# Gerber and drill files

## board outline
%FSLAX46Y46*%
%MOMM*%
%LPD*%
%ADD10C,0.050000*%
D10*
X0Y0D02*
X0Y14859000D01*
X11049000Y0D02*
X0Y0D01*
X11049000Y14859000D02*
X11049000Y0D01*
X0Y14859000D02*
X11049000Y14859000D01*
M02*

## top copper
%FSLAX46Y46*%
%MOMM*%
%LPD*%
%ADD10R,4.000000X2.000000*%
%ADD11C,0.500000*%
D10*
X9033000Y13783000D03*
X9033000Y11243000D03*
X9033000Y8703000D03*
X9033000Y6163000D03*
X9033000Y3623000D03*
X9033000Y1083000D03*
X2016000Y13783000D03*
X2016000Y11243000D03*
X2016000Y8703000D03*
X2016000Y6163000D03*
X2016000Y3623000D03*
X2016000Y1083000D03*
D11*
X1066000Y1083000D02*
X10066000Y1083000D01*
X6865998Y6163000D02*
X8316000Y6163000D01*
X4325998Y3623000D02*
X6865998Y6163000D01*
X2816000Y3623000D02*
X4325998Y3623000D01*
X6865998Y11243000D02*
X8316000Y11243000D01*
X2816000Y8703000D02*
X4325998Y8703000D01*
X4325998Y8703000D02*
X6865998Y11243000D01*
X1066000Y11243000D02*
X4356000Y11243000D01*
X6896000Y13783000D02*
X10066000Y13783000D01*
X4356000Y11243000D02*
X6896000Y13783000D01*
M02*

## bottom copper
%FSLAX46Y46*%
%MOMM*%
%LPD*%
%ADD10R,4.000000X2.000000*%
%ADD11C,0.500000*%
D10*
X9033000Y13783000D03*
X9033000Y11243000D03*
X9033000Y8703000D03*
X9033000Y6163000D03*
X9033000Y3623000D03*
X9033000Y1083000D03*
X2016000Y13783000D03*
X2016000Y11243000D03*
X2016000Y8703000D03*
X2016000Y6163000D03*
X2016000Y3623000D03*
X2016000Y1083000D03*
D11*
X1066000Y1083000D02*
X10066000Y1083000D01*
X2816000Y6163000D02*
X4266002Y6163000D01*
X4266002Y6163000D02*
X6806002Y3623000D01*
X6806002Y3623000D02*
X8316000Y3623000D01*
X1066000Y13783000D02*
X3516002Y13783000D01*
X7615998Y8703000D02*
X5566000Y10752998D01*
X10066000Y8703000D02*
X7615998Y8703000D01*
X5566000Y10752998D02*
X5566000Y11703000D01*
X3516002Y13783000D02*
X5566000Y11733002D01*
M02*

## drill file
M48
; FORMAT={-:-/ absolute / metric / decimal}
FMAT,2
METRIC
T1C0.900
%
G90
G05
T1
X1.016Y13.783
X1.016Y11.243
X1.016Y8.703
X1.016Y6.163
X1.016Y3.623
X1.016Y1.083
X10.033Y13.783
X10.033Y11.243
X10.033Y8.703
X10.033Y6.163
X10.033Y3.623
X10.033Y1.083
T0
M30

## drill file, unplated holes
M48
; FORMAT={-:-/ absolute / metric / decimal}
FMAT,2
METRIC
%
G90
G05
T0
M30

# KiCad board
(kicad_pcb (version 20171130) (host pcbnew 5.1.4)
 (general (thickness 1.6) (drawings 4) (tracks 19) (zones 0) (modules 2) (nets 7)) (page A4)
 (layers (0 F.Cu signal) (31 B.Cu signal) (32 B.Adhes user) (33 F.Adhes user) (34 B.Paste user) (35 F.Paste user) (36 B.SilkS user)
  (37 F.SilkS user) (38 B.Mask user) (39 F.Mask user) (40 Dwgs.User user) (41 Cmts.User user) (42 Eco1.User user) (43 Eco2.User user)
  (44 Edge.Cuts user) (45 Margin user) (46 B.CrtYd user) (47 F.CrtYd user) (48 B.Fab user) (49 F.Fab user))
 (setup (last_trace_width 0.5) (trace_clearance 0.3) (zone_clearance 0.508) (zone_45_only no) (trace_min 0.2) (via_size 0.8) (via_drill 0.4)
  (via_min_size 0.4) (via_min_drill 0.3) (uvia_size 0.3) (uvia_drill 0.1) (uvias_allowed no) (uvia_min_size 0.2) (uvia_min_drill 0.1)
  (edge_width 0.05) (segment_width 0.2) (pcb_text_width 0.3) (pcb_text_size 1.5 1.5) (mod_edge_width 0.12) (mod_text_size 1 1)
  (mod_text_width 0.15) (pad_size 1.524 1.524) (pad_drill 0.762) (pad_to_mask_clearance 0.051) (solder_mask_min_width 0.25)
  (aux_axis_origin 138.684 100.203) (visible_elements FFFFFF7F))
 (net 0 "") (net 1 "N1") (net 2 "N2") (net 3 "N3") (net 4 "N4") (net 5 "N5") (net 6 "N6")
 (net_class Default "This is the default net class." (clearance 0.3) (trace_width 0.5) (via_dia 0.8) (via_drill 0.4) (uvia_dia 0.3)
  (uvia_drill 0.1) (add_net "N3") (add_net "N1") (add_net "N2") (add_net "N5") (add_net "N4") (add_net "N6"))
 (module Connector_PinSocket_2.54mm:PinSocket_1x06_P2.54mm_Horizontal (layer F.Cu) (at 148.717 99.12 180)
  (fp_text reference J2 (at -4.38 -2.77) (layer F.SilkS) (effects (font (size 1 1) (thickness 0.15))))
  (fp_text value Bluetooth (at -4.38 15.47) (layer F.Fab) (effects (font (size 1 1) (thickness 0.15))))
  (pad 6 thru_hole rect (at 0 12.7 180) (size 4 2) (drill 0.9 (offset 1 0)) (layers *.Cu *.Mask) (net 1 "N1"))
  (pad 5 thru_hole rect (at 0 10.16 180) (size 4 2) (drill 0.9 (offset 1 0)) (layers *.Cu *.Mask) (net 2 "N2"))
  (pad 4 thru_hole rect (at 0 7.62 180) (size 4 2) (drill 0.9 (offset 1 0)) (layers *.Cu *.Mask) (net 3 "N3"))
  (pad 3 thru_hole rect (at 0 5.08 180) (size 4 2) (drill 0.9 (offset 1 0)) (layers *.Cu *.Mask) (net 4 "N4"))
  (pad 2 thru_hole rect (at 0 2.54 180) (size 4 2) (drill 0.9 (offset 1 0)) (layers *.Cu *.Mask) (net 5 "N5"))
  (pad 1 thru_hole rect (at 0 0 180) (size 4 2) (drill 0.9 (offset 1 0)) (layers *.Cu *.Mask) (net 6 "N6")))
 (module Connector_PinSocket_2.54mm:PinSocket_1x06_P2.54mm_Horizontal (layer F.Cu) (at 139.7 86.42)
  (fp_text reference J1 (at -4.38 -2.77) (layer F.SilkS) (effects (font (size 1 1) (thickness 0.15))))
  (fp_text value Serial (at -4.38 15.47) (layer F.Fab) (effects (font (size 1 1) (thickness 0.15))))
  (pad 1 thru_hole rect (at 0 0) (size 4 2) (drill 0.9 (offset 1 0)) (layers *.Cu *.Mask) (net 3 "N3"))
  (pad 2 thru_hole rect (at 0 2.54) (size 4 2) (drill 0.9 (offset 1 0)) (layers *.Cu *.Mask) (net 1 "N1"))
  (pad 3 thru_hole rect (at 0 5.08) (size 4 2) (drill 0.9 (offset 1 0)) (layers *.Cu *.Mask) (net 2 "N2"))
  (pad 4 thru_hole rect (at 0 7.62) (size 4 2) (drill 0.9 (offset 1 0)) (layers *.Cu *.Mask) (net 5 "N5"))
  (pad 5 thru_hole rect (at 0 10.16) (size 4 2) (drill 0.9 (offset 1 0)) (layers *.Cu *.Mask) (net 4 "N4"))
  (pad 6 thru_hole rect (at 0 12.7) (size 4 2) (drill 0.9 (offset 1 0)) (layers *.Cu *.Mask) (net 6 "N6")))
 (gr_line (start 138.684 100.203) (end 138.684 85.344) (layer Edge.Cuts) (width 0.05))
 (gr_line (start 149.733 100.203) (end 138.684 100.203) (layer Edge.Cuts) (width 0.05))
 (gr_line (start 149.733 85.344) (end 149.733 100.203) (layer Edge.Cuts) (width 0.05))
 (gr_line (start 138.684 85.344) (end 149.733 85.344) (layer Edge.Cuts) (width 0.05))
 (segment (start 139.75 99.12) (end 148.75 99.12) (width 0.5) (layer F.Cu) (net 6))
 (segment (start 139.75 99.12) (end 148.75 99.12) (width 0.5) (layer B.Cu) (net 6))
 (segment (start 145.549998 94.04) (end 147 94.04) (width 0.5) (layer F.Cu) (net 4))
 (segment (start 143.009998 96.58) (end 145.549998 94.04) (width 0.5) (layer F.Cu) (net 4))
 (segment (start 141.5 96.58) (end 143.009998 96.58) (width 0.5) (layer F.Cu) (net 4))
 (segment (start 141.5 94.04) (end 142.950002 94.04) (width 0.5) (layer B.Cu) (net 5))
 (segment (start 142.950002 94.04) (end 145.490002 96.58) (width 0.5) (layer B.Cu) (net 5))
 (segment (start 145.490002 96.58) (end 147 96.58) (width 0.5) (layer B.Cu) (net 5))
 (segment (start 145.549998 88.96) (end 147 88.96) (width 0.5) (layer F.Cu) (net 2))
 (segment (start 141.5 91.5) (end 143.009998 91.5) (width 0.5) (layer F.Cu) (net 2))
 (segment (start 143.009998 91.5) (end 145.549998 88.96) (width 0.5) (layer F.Cu) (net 2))
 (segment (start 139.75 88.96) (end 143.04 88.96) (width 0.5) (layer F.Cu) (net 1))
 (segment (start 145.58 86.42) (end 148.75 86.42) (width 0.5) (layer F.Cu) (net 1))
 (segment (start 143.04 88.96) (end 145.58 86.42) (width 0.5) (layer F.Cu) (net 1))
 (segment (start 139.75 86.42) (end 142.200002 86.42) (width 0.5) (layer B.Cu) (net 3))
 (segment (start 146.299998 91.5) (end 144.25 89.450002) (width 0.5) (layer B.Cu) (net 3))
 (segment (start 148.75 91.5) (end 146.299998 91.5) (width 0.5) (layer B.Cu) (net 3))
 (segment (start 144.25 89.450002) (end 144.25 88.5) (width 0.5) (layer B.Cu) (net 3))
 (segment (start 142.200002 86.42) (end 144.25 88.469998) (width 0.5) (layer B.Cu) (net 3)))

